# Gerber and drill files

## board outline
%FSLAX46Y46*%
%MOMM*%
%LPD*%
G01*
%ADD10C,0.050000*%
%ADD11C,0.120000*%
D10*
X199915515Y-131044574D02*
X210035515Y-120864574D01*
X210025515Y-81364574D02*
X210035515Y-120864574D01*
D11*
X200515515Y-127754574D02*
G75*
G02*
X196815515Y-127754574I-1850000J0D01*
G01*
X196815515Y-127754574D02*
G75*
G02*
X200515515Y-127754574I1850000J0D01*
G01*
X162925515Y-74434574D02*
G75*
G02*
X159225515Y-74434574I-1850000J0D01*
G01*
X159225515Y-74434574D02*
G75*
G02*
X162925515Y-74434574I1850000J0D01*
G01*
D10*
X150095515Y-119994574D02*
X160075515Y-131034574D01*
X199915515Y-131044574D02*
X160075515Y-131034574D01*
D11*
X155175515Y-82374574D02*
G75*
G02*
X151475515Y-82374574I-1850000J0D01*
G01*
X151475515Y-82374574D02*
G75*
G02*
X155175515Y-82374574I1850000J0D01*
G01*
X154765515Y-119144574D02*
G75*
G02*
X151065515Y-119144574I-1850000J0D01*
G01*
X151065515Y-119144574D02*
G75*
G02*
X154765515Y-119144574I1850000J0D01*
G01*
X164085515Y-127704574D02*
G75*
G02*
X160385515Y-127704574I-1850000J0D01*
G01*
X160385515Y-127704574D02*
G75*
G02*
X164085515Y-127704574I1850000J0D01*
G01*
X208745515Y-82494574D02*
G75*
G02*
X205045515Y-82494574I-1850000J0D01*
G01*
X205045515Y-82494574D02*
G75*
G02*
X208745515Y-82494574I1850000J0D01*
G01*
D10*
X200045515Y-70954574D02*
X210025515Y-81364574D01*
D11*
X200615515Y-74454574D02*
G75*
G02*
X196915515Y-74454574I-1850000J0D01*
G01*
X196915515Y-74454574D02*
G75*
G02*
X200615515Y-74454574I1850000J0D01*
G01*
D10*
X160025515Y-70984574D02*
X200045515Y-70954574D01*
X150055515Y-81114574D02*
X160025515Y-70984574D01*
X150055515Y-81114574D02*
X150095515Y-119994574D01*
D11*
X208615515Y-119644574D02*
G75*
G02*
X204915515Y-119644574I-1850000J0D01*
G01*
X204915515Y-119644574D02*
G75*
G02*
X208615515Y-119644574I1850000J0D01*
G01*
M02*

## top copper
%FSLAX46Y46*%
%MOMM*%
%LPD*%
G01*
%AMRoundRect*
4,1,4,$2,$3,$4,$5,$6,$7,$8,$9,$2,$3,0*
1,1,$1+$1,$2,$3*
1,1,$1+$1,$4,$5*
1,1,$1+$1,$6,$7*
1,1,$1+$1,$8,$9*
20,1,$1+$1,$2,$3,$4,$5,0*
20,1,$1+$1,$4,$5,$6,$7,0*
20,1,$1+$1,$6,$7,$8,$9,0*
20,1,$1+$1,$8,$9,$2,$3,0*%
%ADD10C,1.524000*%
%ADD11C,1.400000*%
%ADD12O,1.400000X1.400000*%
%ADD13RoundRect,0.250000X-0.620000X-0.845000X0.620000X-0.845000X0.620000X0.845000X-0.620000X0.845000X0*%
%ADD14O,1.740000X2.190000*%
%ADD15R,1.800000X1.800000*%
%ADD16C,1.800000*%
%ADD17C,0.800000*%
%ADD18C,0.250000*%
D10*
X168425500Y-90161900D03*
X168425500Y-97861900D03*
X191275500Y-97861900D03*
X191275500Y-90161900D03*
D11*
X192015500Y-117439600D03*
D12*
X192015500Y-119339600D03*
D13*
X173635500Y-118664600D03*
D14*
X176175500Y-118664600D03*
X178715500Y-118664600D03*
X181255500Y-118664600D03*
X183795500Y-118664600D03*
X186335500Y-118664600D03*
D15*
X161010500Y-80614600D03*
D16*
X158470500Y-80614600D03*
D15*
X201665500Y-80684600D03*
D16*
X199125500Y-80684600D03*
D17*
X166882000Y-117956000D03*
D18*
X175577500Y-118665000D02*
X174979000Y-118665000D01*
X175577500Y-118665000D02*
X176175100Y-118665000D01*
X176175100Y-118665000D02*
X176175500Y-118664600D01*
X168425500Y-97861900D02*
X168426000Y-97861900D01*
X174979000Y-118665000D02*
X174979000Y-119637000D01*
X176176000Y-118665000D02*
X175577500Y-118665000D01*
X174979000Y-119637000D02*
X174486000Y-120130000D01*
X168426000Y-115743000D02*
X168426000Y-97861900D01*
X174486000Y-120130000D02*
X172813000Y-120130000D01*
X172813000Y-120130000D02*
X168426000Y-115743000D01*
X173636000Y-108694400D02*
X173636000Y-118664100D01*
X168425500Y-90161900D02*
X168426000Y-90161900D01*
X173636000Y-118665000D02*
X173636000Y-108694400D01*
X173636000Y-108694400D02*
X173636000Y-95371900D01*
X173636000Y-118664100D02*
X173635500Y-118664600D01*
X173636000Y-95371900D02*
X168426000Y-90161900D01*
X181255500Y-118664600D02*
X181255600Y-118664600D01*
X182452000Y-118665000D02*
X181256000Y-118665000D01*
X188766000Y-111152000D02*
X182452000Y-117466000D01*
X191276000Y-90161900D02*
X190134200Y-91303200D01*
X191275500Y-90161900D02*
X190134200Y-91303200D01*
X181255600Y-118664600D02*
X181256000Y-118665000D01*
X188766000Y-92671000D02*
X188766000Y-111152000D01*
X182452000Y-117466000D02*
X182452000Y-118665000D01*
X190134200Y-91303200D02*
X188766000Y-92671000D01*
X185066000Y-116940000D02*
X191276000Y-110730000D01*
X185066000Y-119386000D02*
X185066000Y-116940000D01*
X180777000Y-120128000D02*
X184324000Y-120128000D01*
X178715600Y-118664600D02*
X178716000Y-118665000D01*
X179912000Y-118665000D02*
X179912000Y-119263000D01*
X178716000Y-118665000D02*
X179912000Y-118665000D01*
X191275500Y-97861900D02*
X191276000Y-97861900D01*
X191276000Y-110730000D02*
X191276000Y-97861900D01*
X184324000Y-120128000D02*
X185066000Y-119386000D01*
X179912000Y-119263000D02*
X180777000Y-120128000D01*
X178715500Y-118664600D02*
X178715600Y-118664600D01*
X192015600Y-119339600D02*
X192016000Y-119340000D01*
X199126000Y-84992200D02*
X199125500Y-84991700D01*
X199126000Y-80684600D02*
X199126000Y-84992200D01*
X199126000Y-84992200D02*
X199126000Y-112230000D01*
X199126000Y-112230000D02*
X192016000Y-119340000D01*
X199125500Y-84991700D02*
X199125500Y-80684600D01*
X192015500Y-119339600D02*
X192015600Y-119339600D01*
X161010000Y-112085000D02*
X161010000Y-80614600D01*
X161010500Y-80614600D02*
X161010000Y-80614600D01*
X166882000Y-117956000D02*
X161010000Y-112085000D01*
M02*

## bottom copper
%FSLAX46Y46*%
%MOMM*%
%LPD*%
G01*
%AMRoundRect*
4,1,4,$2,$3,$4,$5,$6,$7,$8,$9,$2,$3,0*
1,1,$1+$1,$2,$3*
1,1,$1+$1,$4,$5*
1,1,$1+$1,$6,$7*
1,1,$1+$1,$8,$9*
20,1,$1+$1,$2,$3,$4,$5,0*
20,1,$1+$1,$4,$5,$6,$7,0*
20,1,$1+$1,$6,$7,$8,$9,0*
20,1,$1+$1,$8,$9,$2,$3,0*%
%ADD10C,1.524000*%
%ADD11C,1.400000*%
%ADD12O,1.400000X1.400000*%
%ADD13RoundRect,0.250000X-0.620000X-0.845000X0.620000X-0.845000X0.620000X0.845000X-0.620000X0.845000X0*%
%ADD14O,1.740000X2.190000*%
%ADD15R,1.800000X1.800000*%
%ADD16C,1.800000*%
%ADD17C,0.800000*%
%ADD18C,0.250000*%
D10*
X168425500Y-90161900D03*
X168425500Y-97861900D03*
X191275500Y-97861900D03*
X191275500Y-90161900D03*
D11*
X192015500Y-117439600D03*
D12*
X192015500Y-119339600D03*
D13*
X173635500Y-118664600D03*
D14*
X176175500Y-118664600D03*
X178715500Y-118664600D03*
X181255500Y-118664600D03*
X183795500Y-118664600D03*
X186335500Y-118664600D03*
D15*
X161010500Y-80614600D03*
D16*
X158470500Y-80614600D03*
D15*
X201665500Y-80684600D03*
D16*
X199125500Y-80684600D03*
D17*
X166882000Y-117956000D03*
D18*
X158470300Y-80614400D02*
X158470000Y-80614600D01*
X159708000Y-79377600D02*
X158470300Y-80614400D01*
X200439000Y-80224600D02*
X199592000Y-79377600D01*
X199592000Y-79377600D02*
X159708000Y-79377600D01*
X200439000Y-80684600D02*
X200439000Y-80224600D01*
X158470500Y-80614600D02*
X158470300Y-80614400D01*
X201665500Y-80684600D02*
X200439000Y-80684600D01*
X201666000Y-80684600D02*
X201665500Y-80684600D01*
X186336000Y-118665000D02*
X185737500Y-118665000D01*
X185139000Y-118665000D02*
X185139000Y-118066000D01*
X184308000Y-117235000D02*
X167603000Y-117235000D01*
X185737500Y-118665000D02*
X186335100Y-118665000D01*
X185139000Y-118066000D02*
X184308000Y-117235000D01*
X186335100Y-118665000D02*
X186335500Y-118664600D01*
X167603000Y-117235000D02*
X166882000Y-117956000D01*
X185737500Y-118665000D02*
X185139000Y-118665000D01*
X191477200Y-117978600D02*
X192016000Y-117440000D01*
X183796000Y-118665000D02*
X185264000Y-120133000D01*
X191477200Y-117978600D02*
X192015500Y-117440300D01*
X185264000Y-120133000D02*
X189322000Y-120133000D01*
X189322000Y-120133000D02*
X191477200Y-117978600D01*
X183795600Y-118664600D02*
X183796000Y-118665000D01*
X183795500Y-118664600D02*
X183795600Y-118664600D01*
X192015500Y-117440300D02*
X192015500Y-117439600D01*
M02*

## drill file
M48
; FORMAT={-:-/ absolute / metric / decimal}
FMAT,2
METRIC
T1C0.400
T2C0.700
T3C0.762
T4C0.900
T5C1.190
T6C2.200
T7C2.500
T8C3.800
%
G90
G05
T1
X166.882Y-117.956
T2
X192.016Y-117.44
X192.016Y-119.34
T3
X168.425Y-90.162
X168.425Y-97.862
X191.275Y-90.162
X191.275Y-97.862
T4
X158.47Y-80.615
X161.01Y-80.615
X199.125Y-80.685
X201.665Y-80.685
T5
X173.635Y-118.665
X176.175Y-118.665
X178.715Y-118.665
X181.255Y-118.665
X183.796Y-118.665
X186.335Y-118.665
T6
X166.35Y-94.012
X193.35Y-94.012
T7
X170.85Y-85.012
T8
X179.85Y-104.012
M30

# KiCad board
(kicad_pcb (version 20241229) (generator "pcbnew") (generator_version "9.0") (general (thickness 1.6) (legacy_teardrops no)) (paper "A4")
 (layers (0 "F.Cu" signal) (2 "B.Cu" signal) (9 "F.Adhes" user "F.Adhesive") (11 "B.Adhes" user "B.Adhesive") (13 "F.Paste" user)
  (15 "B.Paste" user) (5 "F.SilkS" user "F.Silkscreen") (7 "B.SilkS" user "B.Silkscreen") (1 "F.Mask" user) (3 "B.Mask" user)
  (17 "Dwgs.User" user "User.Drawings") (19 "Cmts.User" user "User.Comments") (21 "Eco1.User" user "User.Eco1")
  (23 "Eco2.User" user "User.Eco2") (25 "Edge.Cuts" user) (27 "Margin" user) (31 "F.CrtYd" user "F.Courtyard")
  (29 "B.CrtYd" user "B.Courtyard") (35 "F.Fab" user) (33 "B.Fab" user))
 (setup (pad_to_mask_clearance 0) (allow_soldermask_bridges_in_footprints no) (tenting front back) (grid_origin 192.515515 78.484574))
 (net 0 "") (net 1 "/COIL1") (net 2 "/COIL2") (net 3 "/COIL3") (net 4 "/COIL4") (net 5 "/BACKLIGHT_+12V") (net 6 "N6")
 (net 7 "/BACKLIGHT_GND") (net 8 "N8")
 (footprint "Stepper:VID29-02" (layer "F.Cu") (at 180.0155 94.0119)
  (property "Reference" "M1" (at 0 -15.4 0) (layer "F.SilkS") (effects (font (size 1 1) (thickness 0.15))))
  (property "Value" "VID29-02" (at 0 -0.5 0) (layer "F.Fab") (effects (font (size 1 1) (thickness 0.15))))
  (pad "" np_thru_hole circle (at -13.665 0) (size 2.2 2.2) (drill 2.2) (layers "*.Cu" "*.Mask"))
  (pad "" np_thru_hole circle (at -9.165 -9) (size 2.5 2.5) (drill 2.5) (layers "*.Cu" "*.Mask"))
  (pad "" np_thru_hole circle (at -0.165 10) (size 3.8 3.8) (drill 3.8) (layers "*.Cu" "*.Mask"))
  (pad "" np_thru_hole circle (at 13.335 0) (size 2.2 2.2) (drill 2.2) (layers "*.Cu" "*.Mask"))
  (pad "1" thru_hole circle (at -11.59 -3.85) (size 1.524 1.524) (drill 0.762) (layers "*.Cu" "*.Mask") (remove_unused_layers no)
   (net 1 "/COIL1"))
  (pad "2" thru_hole circle (at -11.59 3.85) (size 1.524 1.524) (drill 0.762) (layers "*.Cu" "*.Mask") (remove_unused_layers no)
   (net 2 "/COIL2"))
  (pad "3" thru_hole circle (at 11.26 3.85) (size 1.524 1.524) (drill 0.762) (layers "*.Cu" "*.Mask") (remove_unused_layers no)
   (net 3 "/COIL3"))
  (pad "4" thru_hole circle (at 11.26 -3.85) (size 1.524 1.524) (drill 0.762) (layers "*.Cu" "*.Mask") (remove_unused_layers no)
   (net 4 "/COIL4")))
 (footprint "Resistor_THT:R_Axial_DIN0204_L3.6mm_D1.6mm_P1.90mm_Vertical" (layer "F.Cu") (at 192.0155 117.4396 -90)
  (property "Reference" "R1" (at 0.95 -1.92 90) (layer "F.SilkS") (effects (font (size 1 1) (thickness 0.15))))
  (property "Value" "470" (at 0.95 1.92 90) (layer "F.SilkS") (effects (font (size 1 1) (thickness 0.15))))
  (pad "1" thru_hole circle (at 0 0 270) (size 1.4 1.4) (drill 0.7) (layers "*.Cu" "*.Mask") (remove_unused_layers no)
   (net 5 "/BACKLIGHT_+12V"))
  (pad "2" thru_hole oval (at 1.9 0 270) (size 1.4 1.4) (drill 0.7) (layers "*.Cu" "*.Mask") (remove_unused_layers no) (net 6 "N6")))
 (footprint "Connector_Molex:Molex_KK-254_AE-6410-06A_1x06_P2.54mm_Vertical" (layer "F.Cu") (at 173.6355 118.6646)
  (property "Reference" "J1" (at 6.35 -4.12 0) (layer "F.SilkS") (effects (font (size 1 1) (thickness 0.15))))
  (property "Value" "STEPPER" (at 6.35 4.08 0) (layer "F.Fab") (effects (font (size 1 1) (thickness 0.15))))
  (pad "1" thru_hole roundrect (at 0 0) (size 1.74 2.19) (drill 1.19) (layers "*.Cu" "*.Mask") (remove_unused_layers no)
   (roundrect_rratio 0.1436781609) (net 1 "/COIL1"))
  (pad "2" thru_hole oval (at 2.54 0) (size 1.74 2.19) (drill 1.19) (layers "*.Cu" "*.Mask") (remove_unused_layers no) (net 2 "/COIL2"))
  (pad "3" thru_hole oval (at 5.08 0) (size 1.74 2.19) (drill 1.19) (layers "*.Cu" "*.Mask") (remove_unused_layers no) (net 3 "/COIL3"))
  (pad "4" thru_hole oval (at 7.62 0) (size 1.74 2.19) (drill 1.19) (layers "*.Cu" "*.Mask") (remove_unused_layers no) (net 4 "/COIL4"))
  (pad "5" thru_hole oval (at 10.16 0) (size 1.74 2.19) (drill 1.19) (layers "*.Cu" "*.Mask") (remove_unused_layers no)
   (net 5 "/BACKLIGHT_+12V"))
  (pad "6" thru_hole oval (at 12.7 0) (size 1.74 2.19) (drill 1.19) (layers "*.Cu" "*.Mask") (remove_unused_layers no)
   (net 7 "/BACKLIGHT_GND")))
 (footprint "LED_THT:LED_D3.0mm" (layer "B.Cu") (at 161.0105 80.6146 180)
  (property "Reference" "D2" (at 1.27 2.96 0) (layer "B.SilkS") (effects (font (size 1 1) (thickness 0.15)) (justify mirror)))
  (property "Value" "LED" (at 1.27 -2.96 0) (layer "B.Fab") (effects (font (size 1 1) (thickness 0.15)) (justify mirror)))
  (pad "1" thru_hole rect (at 0 0 180) (size 1.8 1.8) (drill 0.9) (layers "*.Cu" "*.Mask") (remove_unused_layers no)
   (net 7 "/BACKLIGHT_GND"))
  (pad "2" thru_hole circle (at 2.54 0 180) (size 1.8 1.8) (drill 0.9) (layers "*.Cu" "*.Mask") (remove_unused_layers no) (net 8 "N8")))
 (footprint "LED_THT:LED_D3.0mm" (layer "B.Cu") (at 201.6655 80.6846 180)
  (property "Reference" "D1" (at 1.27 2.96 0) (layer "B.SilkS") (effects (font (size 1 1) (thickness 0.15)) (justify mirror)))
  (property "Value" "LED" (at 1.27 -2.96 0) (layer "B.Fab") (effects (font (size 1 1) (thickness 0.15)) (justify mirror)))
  (pad "1" thru_hole rect (at 0 0 180) (size 1.8 1.8) (drill 0.9) (layers "*.Cu" "*.Mask") (remove_unused_layers no) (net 8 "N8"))
  (pad "2" thru_hole circle (at 2.54 0 180) (size 1.8 1.8) (drill 0.9) (layers "*.Cu" "*.Mask") (remove_unused_layers no) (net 6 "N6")))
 (gr_line (start 199.915515 131.044574) (end 210.035515 120.864574) (stroke (width 0.05) (type solid)) (layer "Edge.Cuts"))
 (gr_line (start 210.025515 81.364574) (end 210.035515 120.864574) (stroke (width 0.05) (type solid)) (layer "Edge.Cuts"))
 (gr_circle (center 198.665515 127.754574) (end 200.515515 127.754574) (stroke (width 0.12) (type solid)) (fill no) (layer "Edge.Cuts"))
 (gr_circle (center 161.075515 74.434574) (end 162.925515 74.434574) (stroke (width 0.12) (type solid)) (fill no) (layer "Edge.Cuts"))
 (gr_line (start 150.095515 119.994574) (end 160.075515 131.034574) (stroke (width 0.05) (type solid)) (layer "Edge.Cuts"))
 (gr_line (start 199.915515 131.044574) (end 160.075515 131.034574) (stroke (width 0.05) (type solid)) (layer "Edge.Cuts"))
 (gr_circle (center 153.325515 82.374574) (end 155.175515 82.374574) (stroke (width 0.12) (type solid)) (fill no) (layer "Edge.Cuts"))
 (gr_circle (center 152.915515 119.144574) (end 154.765515 119.144574) (stroke (width 0.12) (type solid)) (fill no) (layer "Edge.Cuts"))
 (gr_circle (center 162.235515 127.704574) (end 164.085515 127.704574) (stroke (width 0.12) (type solid)) (fill no) (layer "Edge.Cuts"))
 (gr_circle (center 206.895515 82.494574) (end 208.745515 82.494574) (stroke (width 0.12) (type solid)) (fill no) (layer "Edge.Cuts"))
 (gr_line (start 200.045515 70.954574) (end 210.025515 81.364574) (stroke (width 0.05) (type solid)) (layer "Edge.Cuts"))
 (gr_circle (center 198.765515 74.454574) (end 200.615515 74.454574) (stroke (width 0.12) (type solid)) (fill no) (layer "Edge.Cuts"))
 (gr_line (start 160.025515 70.984574) (end 200.045515 70.954574) (stroke (width 0.05) (type solid)) (layer "Edge.Cuts"))
 (gr_line (start 150.055515 81.114574) (end 160.025515 70.984574) (stroke (width 0.05) (type solid)) (layer "Edge.Cuts"))
 (gr_line (start 150.055515 81.114574) (end 150.095515 119.994574) (stroke (width 0.05) (type solid)) (layer "Edge.Cuts"))
 (gr_circle (center 206.765515 119.644574) (end 208.615515 119.644574) (stroke (width 0.12) (type solid)) (fill no) (layer "Edge.Cuts"))
 (segment (start 175.5775 118.665) (end 174.979 118.665) (width 0.25) (layer "F.Cu") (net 2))
 (segment (start 175.5775 118.665) (end 176.1751 118.665) (width 0.25) (layer "F.Cu") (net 2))
 (segment (start 176.1751 118.665) (end 176.1755 118.6646) (width 0.25) (layer "F.Cu") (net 2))
 (segment (start 168.4255 97.8619) (end 168.426 97.8619) (width 0.25) (layer "F.Cu") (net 2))
 (segment (start 174.979 118.665) (end 174.979 119.637) (width 0.25) (layer "F.Cu") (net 2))
 (segment (start 176.176 118.665) (end 175.5775 118.665) (width 0.25) (layer "F.Cu") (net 2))
 (segment (start 174.979 119.637) (end 174.486 120.13) (width 0.25) (layer "F.Cu") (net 2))
 (segment (start 168.426 115.743) (end 168.426 97.8619) (width 0.25) (layer "F.Cu") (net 2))
 (segment (start 174.486 120.13) (end 172.813 120.13) (width 0.25) (layer "F.Cu") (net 2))
 (segment (start 172.813 120.13) (end 168.426 115.743) (width 0.25) (layer "F.Cu") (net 2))
 (segment (start 173.636 108.6944) (end 173.636 118.6641) (width 0.25) (layer "F.Cu") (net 1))
 (segment (start 168.4255 90.1619) (end 168.426 90.1619) (width 0.25) (layer "F.Cu") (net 1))
 (segment (start 173.636 118.665) (end 173.636 108.6944) (width 0.25) (layer "F.Cu") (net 1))
 (segment (start 173.636 108.6944) (end 173.636 95.3719) (width 0.25) (layer "F.Cu") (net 1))
 (segment (start 173.636 118.6641) (end 173.6355 118.6646) (width 0.25) (layer "F.Cu") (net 1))
 (segment (start 173.636 95.3719) (end 168.426 90.1619) (width 0.25) (layer "F.Cu") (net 1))
 (segment (start 181.2555 118.6646) (end 181.2556 118.6646) (width 0.25) (layer "F.Cu") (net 4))
 (segment (start 182.452 118.665) (end 181.256 118.665) (width 0.25) (layer "F.Cu") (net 4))
 (segment (start 188.766 111.152) (end 182.452 117.466) (width 0.25) (layer "F.Cu") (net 4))
 (segment (start 191.276 90.1619) (end 190.1342 91.3032) (width 0.25) (layer "F.Cu") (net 4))
 (segment (start 191.2755 90.1619) (end 190.1342 91.3032) (width 0.25) (layer "F.Cu") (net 4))
 (segment (start 181.2556 118.6646) (end 181.256 118.665) (width 0.25) (layer "F.Cu") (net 4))
 (segment (start 188.766 92.671) (end 188.766 111.152) (width 0.25) (layer "F.Cu") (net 4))
 (segment (start 182.452 117.466) (end 182.452 118.665) (width 0.25) (layer "F.Cu") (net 4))
 (segment (start 190.1342 91.3032) (end 188.766 92.671) (width 0.25) (layer "F.Cu") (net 4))
 (segment (start 185.066 116.94) (end 191.276 110.73) (width 0.25) (layer "F.Cu") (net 3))
 (segment (start 185.066 119.386) (end 185.066 116.94) (width 0.25) (layer "F.Cu") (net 3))
 (segment (start 180.777 120.128) (end 184.324 120.128) (width 0.25) (layer "F.Cu") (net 3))
 (segment (start 178.7156 118.6646) (end 178.716 118.665) (width 0.25) (layer "F.Cu") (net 3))
 (segment (start 179.912 118.665) (end 179.912 119.263) (width 0.25) (layer "F.Cu") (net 3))
 (segment (start 178.716 118.665) (end 179.912 118.665) (width 0.25) (layer "F.Cu") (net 3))
 (segment (start 191.2755 97.8619) (end 191.276 97.8619) (width 0.25) (layer "F.Cu") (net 3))
 (segment (start 191.276 110.73) (end 191.276 97.8619) (width 0.25) (layer "F.Cu") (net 3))
 (segment (start 184.324 120.128) (end 185.066 119.386) (width 0.25) (layer "F.Cu") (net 3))
 (segment (start 179.912 119.263) (end 180.777 120.128) (width 0.25) (layer "F.Cu") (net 3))
 (segment (start 178.7155 118.6646) (end 178.7156 118.6646) (width 0.25) (layer "F.Cu") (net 3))
 (segment (start 192.0156 119.3396) (end 192.016 119.34) (width 0.25) (layer "F.Cu") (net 6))
 (segment (start 199.126 84.9922) (end 199.1255 84.9917) (width 0.25) (layer "F.Cu") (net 6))
 (segment (start 199.126 80.6846) (end 199.126 84.9922) (width 0.25) (layer "F.Cu") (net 6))
 (segment (start 199.126 84.9922) (end 199.126 112.23) (width 0.25) (layer "F.Cu") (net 6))
 (segment (start 199.126 112.23) (end 192.016 119.34) (width 0.25) (layer "F.Cu") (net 6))
 (segment (start 199.1255 84.9917) (end 199.1255 80.6846) (width 0.25) (layer "F.Cu") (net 6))
 (segment (start 192.0155 119.3396) (end 192.0156 119.3396) (width 0.25) (layer "F.Cu") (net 6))
 (segment (start 158.4703 80.6144) (end 158.47 80.6146) (width 0.25) (layer "B.Cu") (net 8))
 (segment (start 159.708 79.3776) (end 158.4703 80.6144) (width 0.25) (layer "B.Cu") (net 8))
 (segment (start 200.439 80.2246) (end 199.592 79.3776) (width 0.25) (layer "B.Cu") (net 8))
 (segment (start 199.592 79.3776) (end 159.708 79.3776) (width 0.25) (layer "B.Cu") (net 8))
 (segment (start 200.439 80.6846) (end 200.439 80.2246) (width 0.25) (layer "B.Cu") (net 8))
 (segment (start 158.4705 80.6146) (end 158.4703 80.6144) (width 0.25) (layer "B.Cu") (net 8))
 (segment (start 201.6655 80.6846) (end 200.439 80.6846) (width 0.25) (layer "B.Cu") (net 8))
 (segment (start 201.666 80.6846) (end 201.6655 80.6846) (width 0.25) (layer "B.Cu") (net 8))
 (segment (start 161.01 112.085) (end 161.01 80.6146) (width 0.25) (layer "F.Cu") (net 7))
 (segment (start 161.0105 80.6146) (end 161.01 80.6146) (width 0.25) (layer "F.Cu") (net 7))
 (segment (start 166.882 117.956) (end 161.01 112.085) (width 0.25) (layer "F.Cu") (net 7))
 (via (at 166.882 117.956) (size 0.8) (drill 0.4) (layers "F.Cu" "B.Cu") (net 7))
 (segment (start 186.336 118.665) (end 185.7375 118.665) (width 0.25) (layer "B.Cu") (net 7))
 (segment (start 185.139 118.665) (end 185.139 118.066) (width 0.25) (layer "B.Cu") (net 7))
 (segment (start 184.308 117.235) (end 167.603 117.235) (width 0.25) (layer "B.Cu") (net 7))
 (segment (start 185.7375 118.665) (end 186.3351 118.665) (width 0.25) (layer "B.Cu") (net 7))
 (segment (start 185.139 118.066) (end 184.308 117.235) (width 0.25) (layer "B.Cu") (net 7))
 (segment (start 186.3351 118.665) (end 186.3355 118.6646) (width 0.25) (layer "B.Cu") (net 7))
 (segment (start 167.603 117.235) (end 166.882 117.956) (width 0.25) (layer "B.Cu") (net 7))
 (segment (start 185.7375 118.665) (end 185.139 118.665) (width 0.25) (layer "B.Cu") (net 7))
 (segment (start 191.4772 117.9786) (end 192.016 117.44) (width 0.25) (layer "B.Cu") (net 5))
 (segment (start 183.796 118.665) (end 185.264 120.133) (width 0.25) (layer "B.Cu") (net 5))
 (segment (start 191.4772 117.9786) (end 192.0155 117.4403) (width 0.25) (layer "B.Cu") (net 5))
 (segment (start 185.264 120.133) (end 189.322 120.133) (width 0.25) (layer "B.Cu") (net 5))
 (segment (start 189.322 120.133) (end 191.4772 117.9786) (width 0.25) (layer "B.Cu") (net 5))
 (segment (start 183.7956 118.6646) (end 183.796 118.665) (width 0.25) (layer "B.Cu") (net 5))
 (segment (start 183.7955 118.6646) (end 183.7956 118.6646) (width 0.25) (layer "B.Cu") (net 5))
 (segment (start 192.0155 117.4403) (end 192.0155 117.4396) (width 0.25) (layer "B.Cu") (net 5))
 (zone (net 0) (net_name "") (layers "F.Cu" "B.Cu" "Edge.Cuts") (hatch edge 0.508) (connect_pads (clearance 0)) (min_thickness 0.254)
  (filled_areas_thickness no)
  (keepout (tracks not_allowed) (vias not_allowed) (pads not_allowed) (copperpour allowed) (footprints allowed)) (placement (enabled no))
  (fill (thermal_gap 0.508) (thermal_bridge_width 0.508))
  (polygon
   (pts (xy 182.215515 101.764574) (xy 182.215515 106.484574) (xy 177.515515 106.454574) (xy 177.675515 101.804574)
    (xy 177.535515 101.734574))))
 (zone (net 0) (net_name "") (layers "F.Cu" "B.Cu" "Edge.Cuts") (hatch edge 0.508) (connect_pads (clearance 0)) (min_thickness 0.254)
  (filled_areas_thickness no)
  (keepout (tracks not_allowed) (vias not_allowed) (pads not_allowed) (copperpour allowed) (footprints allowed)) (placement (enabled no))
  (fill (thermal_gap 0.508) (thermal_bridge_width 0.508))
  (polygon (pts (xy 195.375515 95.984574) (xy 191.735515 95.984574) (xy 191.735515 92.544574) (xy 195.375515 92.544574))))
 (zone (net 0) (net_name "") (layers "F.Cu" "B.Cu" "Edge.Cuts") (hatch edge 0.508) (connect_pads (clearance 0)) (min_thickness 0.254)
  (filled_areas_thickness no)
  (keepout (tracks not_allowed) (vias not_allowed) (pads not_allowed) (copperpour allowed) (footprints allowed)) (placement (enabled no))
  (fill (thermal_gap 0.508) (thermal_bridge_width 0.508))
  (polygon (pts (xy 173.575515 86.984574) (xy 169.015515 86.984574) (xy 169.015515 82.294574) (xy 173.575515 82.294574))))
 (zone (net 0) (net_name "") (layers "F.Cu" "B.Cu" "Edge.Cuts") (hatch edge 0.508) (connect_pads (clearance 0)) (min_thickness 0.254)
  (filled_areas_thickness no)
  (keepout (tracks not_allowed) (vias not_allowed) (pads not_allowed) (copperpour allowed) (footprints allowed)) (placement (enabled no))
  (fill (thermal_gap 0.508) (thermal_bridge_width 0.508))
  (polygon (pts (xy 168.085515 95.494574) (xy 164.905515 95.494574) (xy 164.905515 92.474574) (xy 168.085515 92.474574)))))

